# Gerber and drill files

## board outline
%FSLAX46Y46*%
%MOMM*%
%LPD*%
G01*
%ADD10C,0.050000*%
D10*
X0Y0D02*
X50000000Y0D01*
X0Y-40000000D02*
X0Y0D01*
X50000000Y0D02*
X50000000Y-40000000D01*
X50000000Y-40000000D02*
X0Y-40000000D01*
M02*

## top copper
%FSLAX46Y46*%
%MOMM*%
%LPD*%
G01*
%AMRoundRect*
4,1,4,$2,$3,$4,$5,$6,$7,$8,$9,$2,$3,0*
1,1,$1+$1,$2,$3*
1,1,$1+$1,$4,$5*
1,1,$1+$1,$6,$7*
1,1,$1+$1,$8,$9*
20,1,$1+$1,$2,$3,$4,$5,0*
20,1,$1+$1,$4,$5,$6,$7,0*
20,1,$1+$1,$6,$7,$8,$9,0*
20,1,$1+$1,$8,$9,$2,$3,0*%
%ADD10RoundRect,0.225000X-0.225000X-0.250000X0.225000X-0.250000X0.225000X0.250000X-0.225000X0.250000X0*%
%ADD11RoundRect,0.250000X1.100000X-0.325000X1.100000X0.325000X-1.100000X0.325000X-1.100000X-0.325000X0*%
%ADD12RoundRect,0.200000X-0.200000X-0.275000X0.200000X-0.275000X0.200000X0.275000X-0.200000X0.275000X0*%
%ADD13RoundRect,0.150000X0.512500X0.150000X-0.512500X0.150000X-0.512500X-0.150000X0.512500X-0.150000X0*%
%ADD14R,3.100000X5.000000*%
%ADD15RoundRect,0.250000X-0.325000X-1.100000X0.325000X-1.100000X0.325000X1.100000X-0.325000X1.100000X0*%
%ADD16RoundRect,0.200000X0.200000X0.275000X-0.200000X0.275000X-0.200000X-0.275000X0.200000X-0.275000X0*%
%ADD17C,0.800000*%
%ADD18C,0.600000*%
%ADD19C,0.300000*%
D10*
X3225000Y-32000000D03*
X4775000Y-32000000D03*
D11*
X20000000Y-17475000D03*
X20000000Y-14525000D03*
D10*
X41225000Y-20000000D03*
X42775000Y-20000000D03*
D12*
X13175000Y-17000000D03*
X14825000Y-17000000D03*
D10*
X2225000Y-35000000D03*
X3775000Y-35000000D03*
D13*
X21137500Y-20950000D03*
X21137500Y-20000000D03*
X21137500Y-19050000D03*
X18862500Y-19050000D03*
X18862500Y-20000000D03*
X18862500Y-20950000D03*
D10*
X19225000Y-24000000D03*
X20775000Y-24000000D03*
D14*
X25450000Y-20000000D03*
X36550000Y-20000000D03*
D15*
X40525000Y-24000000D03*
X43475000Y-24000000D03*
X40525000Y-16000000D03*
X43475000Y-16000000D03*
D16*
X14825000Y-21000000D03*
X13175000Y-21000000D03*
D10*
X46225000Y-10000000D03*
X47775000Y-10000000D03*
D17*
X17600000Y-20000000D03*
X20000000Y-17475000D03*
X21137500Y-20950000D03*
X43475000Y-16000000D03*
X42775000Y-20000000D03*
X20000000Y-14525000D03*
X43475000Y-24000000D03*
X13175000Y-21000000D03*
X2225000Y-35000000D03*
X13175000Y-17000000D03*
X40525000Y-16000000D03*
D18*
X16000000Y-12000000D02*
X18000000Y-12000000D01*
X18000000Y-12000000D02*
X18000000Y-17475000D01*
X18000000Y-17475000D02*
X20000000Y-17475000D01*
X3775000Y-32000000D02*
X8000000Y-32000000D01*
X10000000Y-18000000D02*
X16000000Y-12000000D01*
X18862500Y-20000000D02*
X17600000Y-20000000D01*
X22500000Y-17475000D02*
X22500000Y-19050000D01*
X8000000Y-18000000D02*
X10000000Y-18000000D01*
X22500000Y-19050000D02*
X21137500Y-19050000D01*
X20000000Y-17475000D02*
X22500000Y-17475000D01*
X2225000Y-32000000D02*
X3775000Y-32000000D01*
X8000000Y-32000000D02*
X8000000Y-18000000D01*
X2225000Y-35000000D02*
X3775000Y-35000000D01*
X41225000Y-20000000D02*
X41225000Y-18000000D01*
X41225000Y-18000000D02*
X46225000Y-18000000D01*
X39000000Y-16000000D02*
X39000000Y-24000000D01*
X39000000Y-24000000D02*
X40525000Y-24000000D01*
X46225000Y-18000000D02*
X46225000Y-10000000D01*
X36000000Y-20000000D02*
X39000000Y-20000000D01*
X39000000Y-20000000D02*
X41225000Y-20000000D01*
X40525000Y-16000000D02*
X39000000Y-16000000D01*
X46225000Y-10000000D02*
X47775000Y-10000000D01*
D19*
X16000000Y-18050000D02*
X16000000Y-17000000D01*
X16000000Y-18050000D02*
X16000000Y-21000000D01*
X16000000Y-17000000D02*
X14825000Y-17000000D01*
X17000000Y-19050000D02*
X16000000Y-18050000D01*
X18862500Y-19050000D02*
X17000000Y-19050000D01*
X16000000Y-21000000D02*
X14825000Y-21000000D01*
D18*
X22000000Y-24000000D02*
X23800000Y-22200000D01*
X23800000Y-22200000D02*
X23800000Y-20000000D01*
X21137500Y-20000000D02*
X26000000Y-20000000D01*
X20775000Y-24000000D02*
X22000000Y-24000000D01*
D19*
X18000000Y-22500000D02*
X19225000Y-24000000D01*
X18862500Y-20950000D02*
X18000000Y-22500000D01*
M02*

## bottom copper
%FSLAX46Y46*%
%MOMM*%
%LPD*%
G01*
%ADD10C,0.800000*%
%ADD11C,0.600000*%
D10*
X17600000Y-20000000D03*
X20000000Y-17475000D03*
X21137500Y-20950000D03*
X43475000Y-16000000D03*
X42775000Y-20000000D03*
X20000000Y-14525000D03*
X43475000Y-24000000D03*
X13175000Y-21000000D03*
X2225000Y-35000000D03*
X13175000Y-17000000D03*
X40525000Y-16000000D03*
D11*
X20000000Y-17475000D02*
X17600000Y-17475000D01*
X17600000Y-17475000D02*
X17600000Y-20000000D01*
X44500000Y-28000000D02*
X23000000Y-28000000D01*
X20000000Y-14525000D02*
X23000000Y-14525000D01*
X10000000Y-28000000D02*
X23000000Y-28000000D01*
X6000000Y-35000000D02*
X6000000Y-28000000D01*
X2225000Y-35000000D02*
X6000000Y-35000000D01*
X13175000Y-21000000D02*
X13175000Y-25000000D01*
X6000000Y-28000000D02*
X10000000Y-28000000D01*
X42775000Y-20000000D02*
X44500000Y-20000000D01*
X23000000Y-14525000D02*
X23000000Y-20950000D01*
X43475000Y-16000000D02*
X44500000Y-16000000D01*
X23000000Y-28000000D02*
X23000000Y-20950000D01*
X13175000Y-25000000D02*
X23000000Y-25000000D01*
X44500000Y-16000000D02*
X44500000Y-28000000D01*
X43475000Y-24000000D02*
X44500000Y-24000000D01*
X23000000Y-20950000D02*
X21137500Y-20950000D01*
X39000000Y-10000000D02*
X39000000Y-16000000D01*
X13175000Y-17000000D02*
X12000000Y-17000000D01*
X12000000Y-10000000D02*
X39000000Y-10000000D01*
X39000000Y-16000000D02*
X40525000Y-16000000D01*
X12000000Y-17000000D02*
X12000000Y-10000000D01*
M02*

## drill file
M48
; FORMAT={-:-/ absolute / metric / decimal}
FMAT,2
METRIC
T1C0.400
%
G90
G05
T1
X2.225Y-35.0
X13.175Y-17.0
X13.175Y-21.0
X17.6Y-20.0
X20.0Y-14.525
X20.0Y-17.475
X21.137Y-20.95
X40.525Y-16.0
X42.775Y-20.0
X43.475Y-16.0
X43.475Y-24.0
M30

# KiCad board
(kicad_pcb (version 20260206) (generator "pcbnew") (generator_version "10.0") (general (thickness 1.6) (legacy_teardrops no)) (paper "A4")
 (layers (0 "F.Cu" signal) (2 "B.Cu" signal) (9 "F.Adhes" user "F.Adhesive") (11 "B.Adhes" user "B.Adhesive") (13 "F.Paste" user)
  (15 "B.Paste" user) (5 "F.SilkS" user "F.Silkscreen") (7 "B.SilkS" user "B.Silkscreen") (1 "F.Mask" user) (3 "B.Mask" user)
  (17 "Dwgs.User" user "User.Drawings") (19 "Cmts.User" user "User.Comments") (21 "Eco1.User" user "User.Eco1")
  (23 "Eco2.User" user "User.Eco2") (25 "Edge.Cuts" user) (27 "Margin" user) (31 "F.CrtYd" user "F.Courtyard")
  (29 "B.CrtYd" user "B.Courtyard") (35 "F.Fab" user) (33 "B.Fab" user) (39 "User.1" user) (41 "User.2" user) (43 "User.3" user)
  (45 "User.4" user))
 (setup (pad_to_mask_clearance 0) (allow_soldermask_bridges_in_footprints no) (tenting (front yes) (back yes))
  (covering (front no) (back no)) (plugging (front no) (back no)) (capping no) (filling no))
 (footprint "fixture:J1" (layer "F.Cu") (at 4 32)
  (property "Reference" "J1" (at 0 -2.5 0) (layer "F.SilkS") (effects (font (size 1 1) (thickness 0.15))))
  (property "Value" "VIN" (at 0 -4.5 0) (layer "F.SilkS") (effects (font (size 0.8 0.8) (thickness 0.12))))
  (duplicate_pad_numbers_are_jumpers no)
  (pad "1" smd roundrect (at -0.775 0) (size 0.9 0.95) (layers "F.Cu" "F.Mask" "F.Paste") (roundrect_rratio 0.25) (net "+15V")
   (thermal_bridge_angle 45))
  (pad "2" smd roundrect (at 0.775 0) (size 0.9 0.95) (layers "F.Cu" "F.Mask" "F.Paste") (roundrect_rratio 0.25) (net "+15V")
   (thermal_bridge_angle 45)))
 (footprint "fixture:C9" (layer "F.Cu") (at 20 16 90)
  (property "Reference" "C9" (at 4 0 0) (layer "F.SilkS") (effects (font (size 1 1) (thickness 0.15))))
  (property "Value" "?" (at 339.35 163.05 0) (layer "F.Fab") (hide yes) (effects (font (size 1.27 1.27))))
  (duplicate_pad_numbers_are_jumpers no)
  (pad "1" smd roundrect (at -1.475 0 90) (size 1.15 2.7) (layers "F.Cu" "F.Mask" "F.Paste") (roundrect_rratio 0.217391) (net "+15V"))
  (pad "2" smd roundrect (at 1.475 0 90) (size 1.15 2.7) (layers "F.Cu" "F.Mask" "F.Paste") (roundrect_rratio 0.217391) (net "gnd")))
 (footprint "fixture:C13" (layer "F.Cu") (at 42 20)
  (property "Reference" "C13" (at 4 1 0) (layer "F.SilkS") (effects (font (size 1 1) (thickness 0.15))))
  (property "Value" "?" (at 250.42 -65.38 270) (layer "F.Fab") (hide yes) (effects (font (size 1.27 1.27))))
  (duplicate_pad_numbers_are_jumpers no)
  (pad "1" smd roundrect (at -0.775 0) (size 0.9 0.95) (layers "F.Cu" "F.Mask" "F.Paste") (roundrect_rratio 0.25) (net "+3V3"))
  (pad "2" smd roundrect (at 0.775 0) (size 0.9 0.95) (layers "F.Cu" "F.Mask" "F.Paste") (roundrect_rratio 0.25) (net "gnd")))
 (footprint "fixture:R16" (layer "F.Cu") (at 14 17)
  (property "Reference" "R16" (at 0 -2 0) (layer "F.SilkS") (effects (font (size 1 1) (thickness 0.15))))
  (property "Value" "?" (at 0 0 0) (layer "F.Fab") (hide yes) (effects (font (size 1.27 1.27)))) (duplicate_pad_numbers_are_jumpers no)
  (pad "1" smd roundrect (at -0.825 0) (size 0.8 0.95) (layers "F.Cu" "F.Mask" "F.Paste") (roundrect_rratio 0.25) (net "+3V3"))
  (pad "2" smd roundrect (at 0.825 0) (size 0.8 0.95) (layers "F.Cu" "F.Mask" "F.Paste") (roundrect_rratio 0.25) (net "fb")))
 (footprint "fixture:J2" (layer "F.Cu") (at 3 35)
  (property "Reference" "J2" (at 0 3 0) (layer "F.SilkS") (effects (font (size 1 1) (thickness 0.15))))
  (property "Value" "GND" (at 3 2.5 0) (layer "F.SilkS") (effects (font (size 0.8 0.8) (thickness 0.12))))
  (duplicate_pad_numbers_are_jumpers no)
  (pad "1" smd roundrect (at -0.775 0) (size 0.9 0.95) (layers "F.Cu" "F.Mask" "F.Paste") (roundrect_rratio 0.25) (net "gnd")
   (thermal_bridge_angle 45))
  (pad "2" smd roundrect (at 0.775 0) (size 0.9 0.95) (layers "F.Cu" "F.Mask" "F.Paste") (roundrect_rratio 0.25) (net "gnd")
   (thermal_bridge_angle 45)))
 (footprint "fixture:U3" (layer "F.Cu") (at 20 20 180)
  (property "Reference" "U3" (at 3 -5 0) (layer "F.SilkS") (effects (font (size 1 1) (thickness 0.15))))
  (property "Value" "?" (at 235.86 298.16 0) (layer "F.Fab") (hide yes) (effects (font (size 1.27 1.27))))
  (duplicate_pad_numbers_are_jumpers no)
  (pad "1" smd roundrect (at -1.1375 -0.95 180) (size 1.325 0.6) (layers "F.Cu" "F.Mask" "F.Paste") (roundrect_rratio 0.25) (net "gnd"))
  (pad "2" smd roundrect (at -1.1375 0 180) (size 1.325 0.6) (layers "F.Cu" "F.Mask" "F.Paste") (roundrect_rratio 0.25) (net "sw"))
  (pad "3" smd roundrect (at -1.1375 0.95 180) (size 1.325 0.6) (layers "F.Cu" "F.Mask" "F.Paste") (roundrect_rratio 0.25) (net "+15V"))
  (pad "4" smd roundrect (at 1.1375 0.95 180) (size 1.325 0.6) (layers "F.Cu" "F.Mask" "F.Paste") (roundrect_rratio 0.25) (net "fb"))
  (pad "5" smd roundrect (at 1.1375 0 180) (size 1.325 0.6) (layers "F.Cu" "F.Mask" "F.Paste") (roundrect_rratio 0.25) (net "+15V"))
  (pad "6" smd roundrect (at 1.1375 -0.95 180) (size 1.325 0.6) (layers "F.Cu" "F.Mask" "F.Paste") (roundrect_rratio 0.25) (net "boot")))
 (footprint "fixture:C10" (layer "F.Cu") (at 20 24)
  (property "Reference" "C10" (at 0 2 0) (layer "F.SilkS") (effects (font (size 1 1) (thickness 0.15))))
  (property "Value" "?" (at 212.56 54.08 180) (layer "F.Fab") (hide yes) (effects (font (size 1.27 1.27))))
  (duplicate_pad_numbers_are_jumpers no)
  (pad "1" smd roundrect (at -0.775 0) (size 0.9 0.95) (layers "F.Cu" "F.Mask" "F.Paste") (roundrect_rratio 0.25) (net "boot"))
  (pad "2" smd roundrect (at 0.775 0) (size 0.9 0.95) (layers "F.Cu" "F.Mask" "F.Paste") (roundrect_rratio 0.25) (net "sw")))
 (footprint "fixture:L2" (layer "F.Cu") (at 31 20)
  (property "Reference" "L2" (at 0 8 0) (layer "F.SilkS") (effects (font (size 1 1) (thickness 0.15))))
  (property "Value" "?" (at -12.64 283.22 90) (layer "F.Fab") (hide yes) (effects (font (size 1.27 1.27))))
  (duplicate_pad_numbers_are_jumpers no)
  (pad "1" smd rect (at -5.55 0) (size 3.1 5) (layers "F.Cu" "F.Mask" "F.Paste") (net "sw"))
  (pad "2" smd rect (at 5.55 0) (size 3.1 5) (layers "F.Cu" "F.Mask" "F.Paste") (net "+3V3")))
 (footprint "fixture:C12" (layer "F.Cu") (at 42 24)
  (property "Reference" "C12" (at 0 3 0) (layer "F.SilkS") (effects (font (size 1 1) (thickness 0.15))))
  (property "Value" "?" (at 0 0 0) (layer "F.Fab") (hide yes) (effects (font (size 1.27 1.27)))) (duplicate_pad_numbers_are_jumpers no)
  (pad "1" smd roundrect (at -1.475 0) (size 1.15 2.7) (layers "F.Cu" "F.Mask" "F.Paste") (roundrect_rratio 0.217391) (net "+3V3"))
  (pad "2" smd roundrect (at 1.475 0) (size 1.15 2.7) (layers "F.Cu" "F.Mask" "F.Paste") (roundrect_rratio 0.217391) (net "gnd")))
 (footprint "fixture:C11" (layer "F.Cu") (at 42 16)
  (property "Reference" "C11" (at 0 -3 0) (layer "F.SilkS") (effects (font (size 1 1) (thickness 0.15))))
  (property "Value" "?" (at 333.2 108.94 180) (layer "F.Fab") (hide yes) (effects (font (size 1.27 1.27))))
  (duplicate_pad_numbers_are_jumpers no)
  (pad "1" smd roundrect (at -1.475 0) (size 1.15 2.7) (layers "F.Cu" "F.Mask" "F.Paste") (roundrect_rratio 0.217391) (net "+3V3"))
  (pad "2" smd roundrect (at 1.475 0) (size 1.15 2.7) (layers "F.Cu" "F.Mask" "F.Paste") (roundrect_rratio 0.217391) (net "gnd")))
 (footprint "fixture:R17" (layer "F.Cu") (at 14 21 180)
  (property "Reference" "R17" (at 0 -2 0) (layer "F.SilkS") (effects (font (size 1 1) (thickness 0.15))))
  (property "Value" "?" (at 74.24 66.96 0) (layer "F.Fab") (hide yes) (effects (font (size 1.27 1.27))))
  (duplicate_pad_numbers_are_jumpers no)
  (pad "1" smd roundrect (at -0.825 0 180) (size 0.8 0.95) (layers "F.Cu" "F.Mask" "F.Paste") (roundrect_rratio 0.25) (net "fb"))
  (pad "2" smd roundrect (at 0.825 0 180) (size 0.8 0.95) (layers "F.Cu" "F.Mask" "F.Paste") (roundrect_rratio 0.25) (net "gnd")))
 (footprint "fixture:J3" (layer "F.Cu") (at 47 10)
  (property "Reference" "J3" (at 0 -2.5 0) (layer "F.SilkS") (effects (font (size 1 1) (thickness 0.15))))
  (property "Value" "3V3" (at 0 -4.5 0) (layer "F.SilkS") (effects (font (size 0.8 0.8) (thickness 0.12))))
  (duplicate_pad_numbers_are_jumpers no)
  (pad "1" smd roundrect (at -0.775 0) (size 0.9 0.95) (layers "F.Cu" "F.Mask" "F.Paste") (roundrect_rratio 0.25) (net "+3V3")
   (thermal_bridge_angle 45))
  (pad "2" smd roundrect (at 0.775 0) (size 0.9 0.95) (layers "F.Cu" "F.Mask" "F.Paste") (roundrect_rratio 0.25) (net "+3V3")
   (thermal_bridge_angle 45)))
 (gr_line (start 0 0) (end 50 0) (stroke (width 0.05) (type default)) (layer "Edge.Cuts"))
 (gr_line (start 0 40) (end 0 0) (stroke (width 0.05) (type default)) (layer "Edge.Cuts"))
 (gr_line (start 50 0) (end 50 40) (stroke (width 0.05) (type default)) (layer "Edge.Cuts"))
 (gr_line (start 50 40) (end 0 40) (stroke (width 0.05) (type default)) (layer "Edge.Cuts"))
 (segment (start 16 12) (end 18 12) (width 0.6) (layer "F.Cu") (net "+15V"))
 (segment (start 18 12) (end 18 17.475) (width 0.6) (layer "F.Cu") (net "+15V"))
 (segment (start 18 17.475) (end 20 17.475) (width 0.6) (layer "F.Cu") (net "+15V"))
 (segment (start 3.775 32) (end 8 32) (width 0.6) (layer "F.Cu") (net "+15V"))
 (segment (start 10 18) (end 16 12) (width 0.6) (layer "F.Cu") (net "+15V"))
 (segment (start 18.8625 20) (end 17.6 20) (width 0.6) (layer "F.Cu") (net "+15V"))
 (segment (start 22.5 17.475) (end 22.5 19.05) (width 0.6) (layer "F.Cu") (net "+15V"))
 (segment (start 8 18) (end 10 18) (width 0.6) (layer "F.Cu") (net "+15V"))
 (segment (start 22.5 19.05) (end 21.1375 19.05) (width 0.6) (layer "F.Cu") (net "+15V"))
 (segment (start 20 17.475) (end 22.5 17.475) (width 0.6) (layer "F.Cu") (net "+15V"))
 (segment (start 2.225 32) (end 3.775 32) (width 0.6) (layer "F.Cu") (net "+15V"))
 (segment (start 8 32) (end 8 18) (width 0.6) (layer "F.Cu") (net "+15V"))
 (via (at 17.6 20) (size 0.8) (drill 0.4) (layers "F.Cu" "B.Cu") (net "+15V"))
 (via (at 20 17.475) (size 0.8) (drill 0.4) (layers "F.Cu" "B.Cu") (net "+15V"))
 (segment (start 20 17.475) (end 17.6 17.475) (width 0.6) (layer "B.Cu") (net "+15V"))
 (segment (start 17.6 17.475) (end 17.6 20) (width 0.6) (layer "B.Cu") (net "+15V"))
 (segment (start 2.225 35) (end 3.775 35) (width 0.6) (layer "F.Cu") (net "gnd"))
 (via (at 21.1375 20.95) (size 0.8) (drill 0.4) (layers "F.Cu" "B.Cu") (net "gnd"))
 (via (at 43.475 16) (size 0.8) (drill 0.4) (layers "F.Cu" "B.Cu") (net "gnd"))
 (via (at 42.775 20) (size 0.8) (drill 0.4) (layers "F.Cu" "B.Cu") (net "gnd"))
 (via (at 20 14.525) (size 0.8) (drill 0.4) (layers "F.Cu" "B.Cu") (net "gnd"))
 (via (at 43.475 24) (size 0.8) (drill 0.4) (layers "F.Cu" "B.Cu") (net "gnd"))
 (via (at 13.175 21) (size 0.8) (drill 0.4) (layers "F.Cu" "B.Cu") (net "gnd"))
 (via (at 2.225 35) (size 0.8) (drill 0.4) (layers "F.Cu" "B.Cu") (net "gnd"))
 (segment (start 44.5 28) (end 23 28) (width 0.6) (layer "B.Cu") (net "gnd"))
 (segment (start 20 14.525) (end 23 14.525) (width 0.6) (layer "B.Cu") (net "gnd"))
 (segment (start 10 28) (end 23 28) (width 0.6) (layer "B.Cu") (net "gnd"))
 (segment (start 6 35) (end 6 28) (width 0.6) (layer "B.Cu") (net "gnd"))
 (segment (start 2.225 35) (end 6 35) (width 0.6) (layer "B.Cu") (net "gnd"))
 (segment (start 13.175 21) (end 13.175 25) (width 0.6) (layer "B.Cu") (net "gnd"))
 (segment (start 6 28) (end 10 28) (width 0.6) (layer "B.Cu") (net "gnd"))
 (segment (start 42.775 20) (end 44.5 20) (width 0.6) (layer "B.Cu") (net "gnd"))
 (segment (start 23 14.525) (end 23 20.95) (width 0.6) (layer "B.Cu") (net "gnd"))
 (segment (start 43.475 16) (end 44.5 16) (width 0.6) (layer "B.Cu") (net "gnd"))
 (segment (start 23 28) (end 23 20.95) (width 0.6) (layer "B.Cu") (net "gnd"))
 (segment (start 13.175 25) (end 23 25) (width 0.6) (layer "B.Cu") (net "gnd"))
 (segment (start 44.5 16) (end 44.5 28) (width 0.6) (layer "B.Cu") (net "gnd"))
 (segment (start 43.475 24) (end 44.5 24) (width 0.6) (layer "B.Cu") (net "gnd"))
 (segment (start 23 20.95) (end 21.1375 20.95) (width 0.6) (layer "B.Cu") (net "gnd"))
 (segment (start 41.225 20) (end 41.225 18) (width 0.6) (layer "F.Cu") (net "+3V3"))
 (segment (start 41.225 18) (end 46.225 18) (width 0.6) (layer "F.Cu") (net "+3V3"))
 (segment (start 39 16) (end 39 24) (width 0.6) (layer "F.Cu") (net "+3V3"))
 (segment (start 39 24) (end 40.525 24) (width 0.6) (layer "F.Cu") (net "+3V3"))
 (segment (start 46.225 18) (end 46.225 10) (width 0.6) (layer "F.Cu") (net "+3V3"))
 (segment (start 36 20) (end 39 20) (width 0.6) (layer "F.Cu") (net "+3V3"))
 (segment (start 39 20) (end 41.225 20) (width 0.6) (layer "F.Cu") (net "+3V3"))
 (segment (start 40.525 16) (end 39 16) (width 0.6) (layer "F.Cu") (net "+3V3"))
 (segment (start 46.225 10) (end 47.775 10) (width 0.6) (layer "F.Cu") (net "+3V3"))
 (via (at 13.175 17) (size 0.8) (drill 0.4) (layers "F.Cu" "B.Cu") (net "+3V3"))
 (via (at 40.525 16) (size 0.8) (drill 0.4) (layers "F.Cu" "B.Cu") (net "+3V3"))
 (segment (start 39 10) (end 39 16) (width 0.6) (layer "B.Cu") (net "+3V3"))
 (segment (start 13.175 17) (end 12 17) (width 0.6) (layer "B.Cu") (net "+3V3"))
 (segment (start 12 10) (end 39 10) (width 0.6) (layer "B.Cu") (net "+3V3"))
 (segment (start 39 16) (end 40.525 16) (width 0.6) (layer "B.Cu") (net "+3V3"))
 (segment (start 12 17) (end 12 10) (width 0.6) (layer "B.Cu") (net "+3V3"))
 (segment (start 16 18.05) (end 16 17) (width 0.3) (layer "F.Cu") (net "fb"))
 (segment (start 16 18.05) (end 16 21) (width 0.3) (layer "F.Cu") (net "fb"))
 (segment (start 16 17) (end 14.825 17) (width 0.3) (layer "F.Cu") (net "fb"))
 (segment (start 17 19.05) (end 16 18.05) (width 0.3) (layer "F.Cu") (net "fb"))
 (segment (start 18.8625 19.05) (end 17 19.05) (width 0.3) (layer "F.Cu") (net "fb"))
 (segment (start 16 21) (end 14.825 21) (width 0.3) (layer "F.Cu") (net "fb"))
 (segment (start 22 24) (end 23.8 22.2) (width 0.6) (layer "F.Cu") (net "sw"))
 (segment (start 23.8 22.2) (end 23.8 20) (width 0.6) (layer "F.Cu") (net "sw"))
 (segment (start 21.1375 20) (end 26 20) (width 0.6) (layer "F.Cu") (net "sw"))
 (segment (start 20.775 24) (end 22 24) (width 0.6) (layer "F.Cu") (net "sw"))
 (segment (start 18 22.5) (end 19.225 24) (width 0.3) (layer "F.Cu") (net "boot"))
 (segment (start 18.8625 20.95) (end 18 22.5) (width 0.3) (layer "F.Cu") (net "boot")))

